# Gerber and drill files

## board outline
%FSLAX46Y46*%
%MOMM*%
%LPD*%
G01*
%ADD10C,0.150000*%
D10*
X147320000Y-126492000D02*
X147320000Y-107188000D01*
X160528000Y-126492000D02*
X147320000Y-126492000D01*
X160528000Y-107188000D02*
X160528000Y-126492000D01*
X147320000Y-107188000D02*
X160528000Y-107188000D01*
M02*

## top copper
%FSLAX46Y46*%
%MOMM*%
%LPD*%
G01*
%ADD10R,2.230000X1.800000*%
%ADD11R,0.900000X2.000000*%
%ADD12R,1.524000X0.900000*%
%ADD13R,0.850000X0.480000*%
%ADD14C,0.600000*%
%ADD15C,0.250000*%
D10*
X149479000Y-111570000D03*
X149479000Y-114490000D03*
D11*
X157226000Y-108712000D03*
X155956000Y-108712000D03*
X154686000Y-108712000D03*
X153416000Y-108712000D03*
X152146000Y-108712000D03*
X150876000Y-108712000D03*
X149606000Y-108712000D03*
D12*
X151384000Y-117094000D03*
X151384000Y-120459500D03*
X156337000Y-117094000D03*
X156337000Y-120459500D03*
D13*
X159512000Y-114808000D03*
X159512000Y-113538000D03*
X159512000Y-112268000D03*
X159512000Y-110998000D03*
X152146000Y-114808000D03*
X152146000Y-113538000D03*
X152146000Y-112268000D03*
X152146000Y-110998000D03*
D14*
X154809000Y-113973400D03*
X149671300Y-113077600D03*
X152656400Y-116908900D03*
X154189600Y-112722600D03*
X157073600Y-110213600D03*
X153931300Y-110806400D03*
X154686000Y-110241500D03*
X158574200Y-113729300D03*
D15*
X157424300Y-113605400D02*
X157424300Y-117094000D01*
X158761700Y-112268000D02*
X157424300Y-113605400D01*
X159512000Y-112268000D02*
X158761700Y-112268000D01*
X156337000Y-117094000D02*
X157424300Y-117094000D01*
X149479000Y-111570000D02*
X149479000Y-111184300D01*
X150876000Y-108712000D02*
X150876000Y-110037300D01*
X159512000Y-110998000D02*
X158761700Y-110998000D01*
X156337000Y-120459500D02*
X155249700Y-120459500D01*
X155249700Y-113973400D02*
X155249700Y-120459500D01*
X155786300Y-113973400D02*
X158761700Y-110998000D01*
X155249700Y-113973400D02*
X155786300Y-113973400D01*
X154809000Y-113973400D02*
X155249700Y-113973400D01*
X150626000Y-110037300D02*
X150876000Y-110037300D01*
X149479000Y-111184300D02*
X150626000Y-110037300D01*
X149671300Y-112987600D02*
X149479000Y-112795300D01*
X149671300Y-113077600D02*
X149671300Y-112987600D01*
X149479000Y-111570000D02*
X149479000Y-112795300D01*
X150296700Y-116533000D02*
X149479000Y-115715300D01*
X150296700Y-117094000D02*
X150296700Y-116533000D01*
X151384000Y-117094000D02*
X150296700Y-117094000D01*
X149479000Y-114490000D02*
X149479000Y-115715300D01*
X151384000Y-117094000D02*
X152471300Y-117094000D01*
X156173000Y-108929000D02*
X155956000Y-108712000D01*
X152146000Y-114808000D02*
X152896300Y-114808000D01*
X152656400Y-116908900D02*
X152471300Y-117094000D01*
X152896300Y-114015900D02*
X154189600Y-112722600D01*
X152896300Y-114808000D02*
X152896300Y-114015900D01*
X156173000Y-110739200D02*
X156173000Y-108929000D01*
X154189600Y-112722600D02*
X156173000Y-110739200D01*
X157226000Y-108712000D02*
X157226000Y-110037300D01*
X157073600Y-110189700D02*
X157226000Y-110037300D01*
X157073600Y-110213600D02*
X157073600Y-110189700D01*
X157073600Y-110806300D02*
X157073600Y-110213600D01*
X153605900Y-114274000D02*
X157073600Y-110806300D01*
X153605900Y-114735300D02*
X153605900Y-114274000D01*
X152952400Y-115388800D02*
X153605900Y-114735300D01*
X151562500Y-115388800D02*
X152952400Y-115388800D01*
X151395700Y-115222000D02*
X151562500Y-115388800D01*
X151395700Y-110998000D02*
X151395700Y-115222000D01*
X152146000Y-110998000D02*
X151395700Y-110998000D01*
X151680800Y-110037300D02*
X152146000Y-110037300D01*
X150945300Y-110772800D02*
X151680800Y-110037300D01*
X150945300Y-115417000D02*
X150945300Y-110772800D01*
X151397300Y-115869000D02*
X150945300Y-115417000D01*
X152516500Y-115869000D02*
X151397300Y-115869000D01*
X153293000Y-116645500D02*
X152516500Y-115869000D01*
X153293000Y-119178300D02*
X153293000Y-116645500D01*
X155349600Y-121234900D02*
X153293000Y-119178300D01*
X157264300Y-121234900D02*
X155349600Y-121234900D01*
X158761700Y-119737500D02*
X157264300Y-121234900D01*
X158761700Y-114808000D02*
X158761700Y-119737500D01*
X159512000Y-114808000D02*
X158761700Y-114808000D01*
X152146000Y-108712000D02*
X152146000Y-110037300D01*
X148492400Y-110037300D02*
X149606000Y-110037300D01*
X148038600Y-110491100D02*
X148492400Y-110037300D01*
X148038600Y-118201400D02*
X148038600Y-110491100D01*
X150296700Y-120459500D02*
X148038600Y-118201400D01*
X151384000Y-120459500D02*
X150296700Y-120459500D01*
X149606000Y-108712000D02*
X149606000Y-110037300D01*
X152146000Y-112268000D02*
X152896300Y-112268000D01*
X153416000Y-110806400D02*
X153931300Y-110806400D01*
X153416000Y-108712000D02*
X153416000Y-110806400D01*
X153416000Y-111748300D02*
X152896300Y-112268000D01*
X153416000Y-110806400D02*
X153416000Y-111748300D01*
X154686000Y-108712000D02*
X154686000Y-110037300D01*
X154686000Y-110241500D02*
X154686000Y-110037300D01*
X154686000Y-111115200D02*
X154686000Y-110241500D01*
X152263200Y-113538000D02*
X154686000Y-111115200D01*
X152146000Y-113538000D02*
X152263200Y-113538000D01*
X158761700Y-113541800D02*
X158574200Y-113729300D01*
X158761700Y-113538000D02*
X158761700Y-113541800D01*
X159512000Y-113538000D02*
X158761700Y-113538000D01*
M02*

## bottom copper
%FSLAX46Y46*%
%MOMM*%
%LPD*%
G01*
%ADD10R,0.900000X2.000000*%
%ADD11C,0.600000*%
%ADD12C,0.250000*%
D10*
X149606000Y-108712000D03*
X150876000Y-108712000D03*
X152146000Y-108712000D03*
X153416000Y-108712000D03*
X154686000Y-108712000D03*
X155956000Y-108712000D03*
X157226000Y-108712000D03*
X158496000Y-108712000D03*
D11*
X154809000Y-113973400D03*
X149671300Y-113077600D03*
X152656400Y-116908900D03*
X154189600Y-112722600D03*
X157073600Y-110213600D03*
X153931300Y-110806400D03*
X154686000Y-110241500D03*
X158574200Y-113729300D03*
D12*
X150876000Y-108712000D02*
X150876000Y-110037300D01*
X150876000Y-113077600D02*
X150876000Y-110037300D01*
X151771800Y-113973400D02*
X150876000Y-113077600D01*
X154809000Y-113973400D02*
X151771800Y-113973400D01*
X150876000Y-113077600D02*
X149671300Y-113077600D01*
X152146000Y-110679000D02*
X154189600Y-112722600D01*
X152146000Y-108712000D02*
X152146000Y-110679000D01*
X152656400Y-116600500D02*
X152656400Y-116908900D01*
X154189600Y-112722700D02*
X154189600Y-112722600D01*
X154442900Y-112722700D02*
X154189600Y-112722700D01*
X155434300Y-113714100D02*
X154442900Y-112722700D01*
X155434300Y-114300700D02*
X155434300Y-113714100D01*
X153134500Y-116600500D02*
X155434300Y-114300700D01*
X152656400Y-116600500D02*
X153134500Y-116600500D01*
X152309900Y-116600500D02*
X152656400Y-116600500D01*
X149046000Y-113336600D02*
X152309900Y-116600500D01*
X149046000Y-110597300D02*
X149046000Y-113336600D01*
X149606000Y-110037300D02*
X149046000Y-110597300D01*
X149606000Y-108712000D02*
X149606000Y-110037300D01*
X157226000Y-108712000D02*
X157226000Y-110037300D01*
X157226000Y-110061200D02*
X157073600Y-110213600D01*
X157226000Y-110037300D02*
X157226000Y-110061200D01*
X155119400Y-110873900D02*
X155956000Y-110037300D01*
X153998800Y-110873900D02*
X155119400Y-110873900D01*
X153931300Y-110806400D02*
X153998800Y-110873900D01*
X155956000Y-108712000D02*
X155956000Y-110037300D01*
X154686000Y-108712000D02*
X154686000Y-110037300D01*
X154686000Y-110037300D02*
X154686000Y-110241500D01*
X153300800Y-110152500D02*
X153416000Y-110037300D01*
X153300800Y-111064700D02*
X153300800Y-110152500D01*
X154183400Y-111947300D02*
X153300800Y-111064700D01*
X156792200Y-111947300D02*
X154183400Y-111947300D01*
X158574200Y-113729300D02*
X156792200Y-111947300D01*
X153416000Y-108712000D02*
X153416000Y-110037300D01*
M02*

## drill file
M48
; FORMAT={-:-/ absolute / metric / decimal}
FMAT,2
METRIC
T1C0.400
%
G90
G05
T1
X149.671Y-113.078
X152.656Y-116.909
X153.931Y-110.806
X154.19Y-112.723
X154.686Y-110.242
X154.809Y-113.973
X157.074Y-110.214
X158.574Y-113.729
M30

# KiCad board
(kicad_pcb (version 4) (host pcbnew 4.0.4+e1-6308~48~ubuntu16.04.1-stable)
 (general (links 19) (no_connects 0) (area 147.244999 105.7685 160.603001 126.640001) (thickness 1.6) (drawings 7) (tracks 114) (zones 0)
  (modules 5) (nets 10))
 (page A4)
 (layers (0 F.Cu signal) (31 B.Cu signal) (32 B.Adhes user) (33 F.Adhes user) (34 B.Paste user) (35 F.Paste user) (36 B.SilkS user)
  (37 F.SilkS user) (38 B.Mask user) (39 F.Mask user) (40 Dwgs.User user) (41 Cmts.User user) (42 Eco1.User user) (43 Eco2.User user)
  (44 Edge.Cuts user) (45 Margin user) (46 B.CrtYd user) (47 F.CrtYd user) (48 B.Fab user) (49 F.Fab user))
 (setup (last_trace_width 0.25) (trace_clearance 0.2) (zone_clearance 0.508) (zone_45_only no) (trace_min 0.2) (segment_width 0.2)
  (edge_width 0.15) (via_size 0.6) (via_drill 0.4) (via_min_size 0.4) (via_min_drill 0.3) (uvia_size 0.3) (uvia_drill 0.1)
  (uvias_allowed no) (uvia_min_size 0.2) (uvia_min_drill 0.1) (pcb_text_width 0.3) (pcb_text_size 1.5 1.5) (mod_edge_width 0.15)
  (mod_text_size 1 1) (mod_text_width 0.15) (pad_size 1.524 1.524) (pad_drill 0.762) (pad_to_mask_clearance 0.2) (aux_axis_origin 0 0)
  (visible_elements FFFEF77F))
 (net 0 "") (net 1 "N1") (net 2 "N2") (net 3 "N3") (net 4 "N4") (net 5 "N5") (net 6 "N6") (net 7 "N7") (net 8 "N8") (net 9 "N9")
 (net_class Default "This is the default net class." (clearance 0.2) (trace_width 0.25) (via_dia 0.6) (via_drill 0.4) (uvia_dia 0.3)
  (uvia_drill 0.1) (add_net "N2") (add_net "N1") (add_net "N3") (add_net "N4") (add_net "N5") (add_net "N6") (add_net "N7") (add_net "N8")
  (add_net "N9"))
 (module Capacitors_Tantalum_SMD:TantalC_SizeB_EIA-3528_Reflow (layer F.Cu) (at 149.479 113.03 90)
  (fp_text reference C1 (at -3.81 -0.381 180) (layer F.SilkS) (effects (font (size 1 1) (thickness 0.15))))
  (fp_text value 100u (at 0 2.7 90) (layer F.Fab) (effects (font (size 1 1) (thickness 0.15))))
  (pad 2 smd rect (at 1.46 0 90) (size 1.8 2.23) (layers F.Cu F.Paste F.Mask) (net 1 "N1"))
  (pad 1 smd rect (at -1.46 0 90) (size 1.8 2.23) (layers F.Cu F.Paste F.Mask) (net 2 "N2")))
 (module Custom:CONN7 (layer F.Cu) (at 157.226 108.712 180)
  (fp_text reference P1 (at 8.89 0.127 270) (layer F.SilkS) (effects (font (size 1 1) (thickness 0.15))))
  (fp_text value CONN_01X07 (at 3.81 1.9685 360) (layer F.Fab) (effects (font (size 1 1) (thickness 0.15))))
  (pad 1 smd rect (at 0 0 180) (size 0.9 2) (layers F.Cu F.Paste F.Mask) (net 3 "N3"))
  (pad 2 smd rect (at 1.27 0 180) (size 0.9 2) (layers F.Cu F.Paste F.Mask) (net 2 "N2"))
  (pad 3 smd rect (at 2.54 0 180) (size 0.9 2) (layers F.Cu F.Paste F.Mask) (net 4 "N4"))
  (pad 4 smd rect (at 3.81 0 180) (size 0.9 2) (layers F.Cu F.Paste F.Mask) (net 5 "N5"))
  (pad 5 smd rect (at 5.08 0 180) (size 0.9 2) (layers F.Cu F.Paste F.Mask) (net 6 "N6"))
  (pad 6 smd rect (at 6.35 0 180) (size 0.9 2) (layers F.Cu F.Paste F.Mask) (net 1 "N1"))
  (pad 7 smd rect (at 7.62 0 180) (size 0.9 2) (layers F.Cu F.Paste F.Mask) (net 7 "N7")))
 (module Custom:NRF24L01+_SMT (layer B.Cu) (at 149.606 108.712)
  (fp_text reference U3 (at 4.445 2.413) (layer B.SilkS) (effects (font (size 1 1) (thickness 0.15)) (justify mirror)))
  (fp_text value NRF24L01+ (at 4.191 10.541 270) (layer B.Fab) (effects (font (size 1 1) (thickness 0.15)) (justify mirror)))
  (pad 1 smd rect (at 0 0) (size 0.9 2) (layers B.Cu B.Paste B.Mask) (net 2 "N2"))
  (pad 2 smd rect (at 1.27 0) (size 0.9 2) (layers B.Cu B.Paste B.Mask) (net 1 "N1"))
  (pad 3 smd rect (at 2.54 0) (size 0.9 2) (layers B.Cu B.Paste B.Mask) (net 2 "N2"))
  (pad 4 smd rect (at 3.81 0) (size 0.9 2) (layers B.Cu B.Paste B.Mask) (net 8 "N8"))
  (pad 5 smd rect (at 5.08 0) (size 0.9 2) (layers B.Cu B.Paste B.Mask) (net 4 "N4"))
  (pad 6 smd rect (at 6.35 0) (size 0.9 2) (layers B.Cu B.Paste B.Mask) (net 5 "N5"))
  (pad 7 smd rect (at 7.62 0) (size 0.9 2) (layers B.Cu B.Paste B.Mask) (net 3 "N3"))
  (pad 8 smd rect (at 8.89 0) (size 0.9 2) (layers B.Cu B.Paste B.Mask)))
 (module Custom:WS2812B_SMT (layer F.Cu) (at 151.384 117.094)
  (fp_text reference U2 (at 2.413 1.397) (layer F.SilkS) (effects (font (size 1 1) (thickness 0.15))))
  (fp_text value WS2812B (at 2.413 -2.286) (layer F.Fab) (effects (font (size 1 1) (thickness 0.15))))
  (pad 1 smd rect (at 0 0) (size 1.524 0.9) (layers F.Cu F.Paste F.Mask) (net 2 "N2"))
  (pad 2 smd rect (at 0 3.3655) (size 1.524 0.9) (layers F.Cu F.Paste F.Mask) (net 7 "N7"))
  (pad 4 smd rect (at 4.953 0) (size 1.524 0.9) (layers F.Cu F.Paste F.Mask) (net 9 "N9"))
  (pad 3 smd rect (at 4.953 3.3655) (size 1.524 0.9) (layers F.Cu F.Paste F.Mask) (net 1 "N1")))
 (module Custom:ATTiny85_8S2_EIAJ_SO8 (layer F.Cu) (at 159.512 114.808 180)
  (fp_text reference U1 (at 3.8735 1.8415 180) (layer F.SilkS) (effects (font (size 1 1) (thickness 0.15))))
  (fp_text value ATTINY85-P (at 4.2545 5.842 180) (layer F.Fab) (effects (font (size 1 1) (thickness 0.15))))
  (pad 1 smd rect (at 0 0 180) (size 0.85 0.48) (layers F.Cu F.Paste F.Mask) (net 6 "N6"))
  (pad 2 smd rect (at 0 1.27 180) (size 0.85 0.48) (layers F.Cu F.Paste F.Mask) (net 8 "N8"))
  (pad 3 smd rect (at 0 2.54 180) (size 0.85 0.48) (layers F.Cu F.Paste F.Mask) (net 9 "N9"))
  (pad 4 smd rect (at 0 3.81 180) (size 0.85 0.48) (layers F.Cu F.Paste F.Mask) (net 1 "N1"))
  (pad 8 smd rect (at 7.366 0 180) (size 0.85 0.48) (layers F.Cu F.Paste F.Mask) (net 2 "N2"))
  (pad 7 smd rect (at 7.366 1.27 180) (size 0.85 0.48) (layers F.Cu F.Paste F.Mask) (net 4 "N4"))
  (pad 6 smd rect (at 7.366 2.54 180) (size 0.85 0.48) (layers F.Cu F.Paste F.Mask) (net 5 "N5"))
  (pad 5 smd rect (at 7.366 3.81 180) (size 0.85 0.48) (layers F.Cu F.Paste F.Mask) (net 3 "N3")))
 (gr_line (start 147.32 126.492) (end 147.32 107.188) (angle 90) (layer Edge.Cuts) (width 0.15))
 (gr_line (start 160.528 126.492) (end 147.32 126.492) (angle 90) (layer Edge.Cuts) (width 0.15))
 (gr_line (start 160.528 107.188) (end 160.528 126.492) (angle 90) (layer Edge.Cuts) (width 0.15))
 (gr_line (start 147.32 107.188) (end 160.528 107.188) (angle 90) (layer Edge.Cuts) (width 0.15))
 (segment (start 157.4243 113.6054) (end 157.4243 117.094) (width 0.25) (layer F.Cu) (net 9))
 (segment (start 158.7617 112.268) (end 157.4243 113.6054) (width 0.25) (layer F.Cu) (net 9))
 (segment (start 159.512 112.268) (end 158.7617 112.268) (width 0.25) (layer F.Cu) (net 9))
 (segment (start 156.337 117.094) (end 157.4243 117.094) (width 0.25) (layer F.Cu) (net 9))
 (via (at 154.809 113.9734) (size 0.6) (layers F.Cu B.Cu) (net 1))
 (via (at 149.6713 113.0776) (size 0.6) (layers F.Cu B.Cu) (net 1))
 (segment (start 149.479 111.57) (end 149.479 111.1843) (width 0.25) (layer F.Cu) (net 1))
 (segment (start 150.876 108.712) (end 150.876 110.0373) (width 0.25) (layer F.Cu) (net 1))
 (segment (start 150.876 108.712) (end 150.876 110.0373) (width 0.25) (layer B.Cu) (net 1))
 (segment (start 159.512 110.998) (end 158.7617 110.998) (width 0.25) (layer F.Cu) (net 1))
 (segment (start 156.337 120.4595) (end 155.2497 120.4595) (width 0.25) (layer F.Cu) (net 1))
 (segment (start 155.2497 113.9734) (end 155.2497 120.4595) (width 0.25) (layer F.Cu) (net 1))
 (segment (start 155.7863 113.9734) (end 158.7617 110.998) (width 0.25) (layer F.Cu) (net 1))
 (segment (start 155.2497 113.9734) (end 155.7863 113.9734) (width 0.25) (layer F.Cu) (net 1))
 (segment (start 154.809 113.9734) (end 155.2497 113.9734) (width 0.25) (layer F.Cu) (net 1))
 (segment (start 150.626 110.0373) (end 150.876 110.0373) (width 0.25) (layer F.Cu) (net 1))
 (segment (start 149.479 111.1843) (end 150.626 110.0373) (width 0.25) (layer F.Cu) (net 1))
 (segment (start 149.6713 112.9876) (end 149.479 112.7953) (width 0.25) (layer F.Cu) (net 1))
 (segment (start 149.6713 113.0776) (end 149.6713 112.9876) (width 0.25) (layer F.Cu) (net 1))
 (segment (start 149.479 111.57) (end 149.479 112.7953) (width 0.25) (layer F.Cu) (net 1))
 (segment (start 150.876 113.0776) (end 150.876 110.0373) (width 0.25) (layer B.Cu) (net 1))
 (segment (start 151.7718 113.9734) (end 150.876 113.0776) (width 0.25) (layer B.Cu) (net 1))
 (segment (start 154.809 113.9734) (end 151.7718 113.9734) (width 0.25) (layer B.Cu) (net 1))
 (segment (start 150.876 113.0776) (end 149.6713 113.0776) (width 0.25) (layer B.Cu) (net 1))
 (via (at 152.6564 116.9089) (size 0.6) (layers F.Cu B.Cu) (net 2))
 (via (at 154.1896 112.7226) (size 0.6) (layers F.Cu B.Cu) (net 2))
 (segment (start 150.2967 116.533) (end 149.479 115.7153) (width 0.25) (layer F.Cu) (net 2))
 (segment (start 150.2967 117.094) (end 150.2967 116.533) (width 0.25) (layer F.Cu) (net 2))
 (segment (start 151.384 117.094) (end 150.2967 117.094) (width 0.25) (layer F.Cu) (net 2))
 (segment (start 149.479 114.49) (end 149.479 115.7153) (width 0.25) (layer F.Cu) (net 2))
 (segment (start 151.384 117.094) (end 152.4713 117.094) (width 0.25) (layer F.Cu) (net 2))
 (segment (start 156.173 108.929) (end 155.956 108.712) (width 0.25) (layer F.Cu) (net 2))
 (segment (start 152.146 114.808) (end 152.8963 114.808) (width 0.25) (layer F.Cu) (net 2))
 (segment (start 152.6564 116.9089) (end 152.4713 117.094) (width 0.25) (layer F.Cu) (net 2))
 (segment (start 152.8963 114.0159) (end 154.1896 112.7226) (width 0.25) (layer F.Cu) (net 2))
 (segment (start 152.8963 114.808) (end 152.8963 114.0159) (width 0.25) (layer F.Cu) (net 2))
 (segment (start 156.173 110.7392) (end 156.173 108.929) (width 0.25) (layer F.Cu) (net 2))
 (segment (start 154.1896 112.7226) (end 156.173 110.7392) (width 0.25) (layer F.Cu) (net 2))
 (segment (start 152.146 110.679) (end 154.1896 112.7226) (width 0.25) (layer B.Cu) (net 2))
 (segment (start 152.146 108.712) (end 152.146 110.679) (width 0.25) (layer B.Cu) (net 2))
 (segment (start 152.6564 116.6005) (end 152.6564 116.9089) (width 0.25) (layer B.Cu) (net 2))
 (segment (start 154.1896 112.7227) (end 154.1896 112.7226) (width 0.25) (layer B.Cu) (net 2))
 (segment (start 154.4429 112.7227) (end 154.1896 112.7227) (width 0.25) (layer B.Cu) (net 2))
 (segment (start 155.4343 113.7141) (end 154.4429 112.7227) (width 0.25) (layer B.Cu) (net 2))
 (segment (start 155.4343 114.3007) (end 155.4343 113.7141) (width 0.25) (layer B.Cu) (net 2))
 (segment (start 153.1345 116.6005) (end 155.4343 114.3007) (width 0.25) (layer B.Cu) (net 2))
 (segment (start 152.6564 116.6005) (end 153.1345 116.6005) (width 0.25) (layer B.Cu) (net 2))
 (segment (start 152.3099 116.6005) (end 152.6564 116.6005) (width 0.25) (layer B.Cu) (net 2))
 (segment (start 149.046 113.3366) (end 152.3099 116.6005) (width 0.25) (layer B.Cu) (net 2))
 (segment (start 149.046 110.5973) (end 149.046 113.3366) (width 0.25) (layer B.Cu) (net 2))
 (segment (start 149.606 110.0373) (end 149.046 110.5973) (width 0.25) (layer B.Cu) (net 2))
 (segment (start 149.606 108.712) (end 149.606 110.0373) (width 0.25) (layer B.Cu) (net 2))
 (via (at 157.0736 110.2136) (size 0.6) (layers F.Cu B.Cu) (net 3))
 (segment (start 157.226 108.712) (end 157.226 110.0373) (width 0.25) (layer B.Cu) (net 3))
 (segment (start 157.226 108.712) (end 157.226 110.0373) (width 0.25) (layer F.Cu) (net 3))
 (segment (start 157.0736 110.1897) (end 157.226 110.0373) (width 0.25) (layer F.Cu) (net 3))
 (segment (start 157.0736 110.2136) (end 157.0736 110.1897) (width 0.25) (layer F.Cu) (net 3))
 (segment (start 157.226 110.0612) (end 157.0736 110.2136) (width 0.25) (layer B.Cu) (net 3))
 (segment (start 157.226 110.0373) (end 157.226 110.0612) (width 0.25) (layer B.Cu) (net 3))
 (segment (start 157.0736 110.8063) (end 157.0736 110.2136) (width 0.25) (layer F.Cu) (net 3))
 (segment (start 153.6059 114.274) (end 157.0736 110.8063) (width 0.25) (layer F.Cu) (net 3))
 (segment (start 153.6059 114.7353) (end 153.6059 114.274) (width 0.25) (layer F.Cu) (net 3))
 (segment (start 152.9524 115.3888) (end 153.6059 114.7353) (width 0.25) (layer F.Cu) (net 3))
 (segment (start 151.5625 115.3888) (end 152.9524 115.3888) (width 0.25) (layer F.Cu) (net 3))
 (segment (start 151.3957 115.222) (end 151.5625 115.3888) (width 0.25) (layer F.Cu) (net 3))
 (segment (start 151.3957 110.998) (end 151.3957 115.222) (width 0.25) (layer F.Cu) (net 3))
 (segment (start 152.146 110.998) (end 151.3957 110.998) (width 0.25) (layer F.Cu) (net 3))
 (segment (start 151.6808 110.0373) (end 152.146 110.0373) (width 0.25) (layer F.Cu) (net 6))
 (segment (start 150.9453 110.7728) (end 151.6808 110.0373) (width 0.25) (layer F.Cu) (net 6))
 (segment (start 150.9453 115.417) (end 150.9453 110.7728) (width 0.25) (layer F.Cu) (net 6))
 (segment (start 151.3973 115.869) (end 150.9453 115.417) (width 0.25) (layer F.Cu) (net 6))
 (segment (start 152.5165 115.869) (end 151.3973 115.869) (width 0.25) (layer F.Cu) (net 6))
 (segment (start 153.293 116.6455) (end 152.5165 115.869) (width 0.25) (layer F.Cu) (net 6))
 (segment (start 153.293 119.1783) (end 153.293 116.6455) (width 0.25) (layer F.Cu) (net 6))
 (segment (start 155.3496 121.2349) (end 153.293 119.1783) (width 0.25) (layer F.Cu) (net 6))
 (segment (start 157.2643 121.2349) (end 155.3496 121.2349) (width 0.25) (layer F.Cu) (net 6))
 (segment (start 158.7617 119.7375) (end 157.2643 121.2349) (width 0.25) (layer F.Cu) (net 6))
 (segment (start 158.7617 114.808) (end 158.7617 119.7375) (width 0.25) (layer F.Cu) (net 6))
 (segment (start 159.512 114.808) (end 158.7617 114.808) (width 0.25) (layer F.Cu) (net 6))
 (segment (start 152.146 108.712) (end 152.146 110.0373) (width 0.25) (layer F.Cu) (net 6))
 (segment (start 148.4924 110.0373) (end 149.606 110.0373) (width 0.25) (layer F.Cu) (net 7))
 (segment (start 148.0386 110.4911) (end 148.4924 110.0373) (width 0.25) (layer F.Cu) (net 7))
 (segment (start 148.0386 118.2014) (end 148.0386 110.4911) (width 0.25) (layer F.Cu) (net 7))
 (segment (start 150.2967 120.4595) (end 148.0386 118.2014) (width 0.25) (layer F.Cu) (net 7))
 (segment (start 151.384 120.4595) (end 150.2967 120.4595) (width 0.25) (layer F.Cu) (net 7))
 (segment (start 149.606 108.712) (end 149.606 110.0373) (width 0.25) (layer F.Cu) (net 7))
 (via (at 153.9313 110.8064) (size 0.6) (layers F.Cu B.Cu) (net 5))
 (segment (start 152.146 112.268) (end 152.8963 112.268) (width 0.25) (layer F.Cu) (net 5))
 (segment (start 155.1194 110.8739) (end 155.956 110.0373) (width 0.25) (layer B.Cu) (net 5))
 (segment (start 153.9988 110.8739) (end 155.1194 110.8739) (width 0.25) (layer B.Cu) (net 5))
 (segment (start 153.9313 110.8064) (end 153.9988 110.8739) (width 0.25) (layer B.Cu) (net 5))
 (segment (start 153.416 110.8064) (end 153.9313 110.8064) (width 0.25) (layer F.Cu) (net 5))
 (segment (start 153.416 108.712) (end 153.416 110.8064) (width 0.25) (layer F.Cu) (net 5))
 (segment (start 153.416 111.7483) (end 152.8963 112.268) (width 0.25) (layer F.Cu) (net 5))
 (segment (start 153.416 110.8064) (end 153.416 111.7483) (width 0.25) (layer F.Cu) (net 5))
 (segment (start 155.956 108.712) (end 155.956 110.0373) (width 0.25) (layer B.Cu) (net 5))
 (via (at 154.686 110.2415) (size 0.6) (layers F.Cu B.Cu) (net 4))
 (segment (start 154.686 108.712) (end 154.686 110.0373) (width 0.25) (layer F.Cu) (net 4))
 (segment (start 154.686 108.712) (end 154.686 110.0373) (width 0.25) (layer B.Cu) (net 4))
 (segment (start 154.686 110.0373) (end 154.686 110.2415) (width 0.25) (layer B.Cu) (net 4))
 (segment (start 154.686 110.2415) (end 154.686 110.0373) (width 0.25) (layer F.Cu) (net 4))
 (segment (start 154.686 111.1152) (end 154.686 110.2415) (width 0.25) (layer F.Cu) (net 4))
 (segment (start 152.2632 113.538) (end 154.686 111.1152) (width 0.25) (layer F.Cu) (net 4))
 (segment (start 152.146 113.538) (end 152.2632 113.538) (width 0.25) (layer F.Cu) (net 4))
 (via (at 158.5742 113.7293) (size 0.6) (layers F.Cu B.Cu) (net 8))
 (segment (start 158.7617 113.5418) (end 158.5742 113.7293) (width 0.25) (layer F.Cu) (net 8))
 (segment (start 158.7617 113.538) (end 158.7617 113.5418) (width 0.25) (layer F.Cu) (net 8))
 (segment (start 153.3008 110.1525) (end 153.416 110.0373) (width 0.25) (layer B.Cu) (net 8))
 (segment (start 153.3008 111.0647) (end 153.3008 110.1525) (width 0.25) (layer B.Cu) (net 8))
 (segment (start 154.1834 111.9473) (end 153.3008 111.0647) (width 0.25) (layer B.Cu) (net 8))
 (segment (start 156.7922 111.9473) (end 154.1834 111.9473) (width 0.25) (layer B.Cu) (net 8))
 (segment (start 158.5742 113.7293) (end 156.7922 111.9473) (width 0.25) (layer B.Cu) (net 8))
 (segment (start 159.512 113.538) (end 158.7617 113.538) (width 0.25) (layer F.Cu) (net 8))
 (segment (start 153.416 108.712) (end 153.416 110.0373) (width 0.25) (layer B.Cu) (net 8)))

